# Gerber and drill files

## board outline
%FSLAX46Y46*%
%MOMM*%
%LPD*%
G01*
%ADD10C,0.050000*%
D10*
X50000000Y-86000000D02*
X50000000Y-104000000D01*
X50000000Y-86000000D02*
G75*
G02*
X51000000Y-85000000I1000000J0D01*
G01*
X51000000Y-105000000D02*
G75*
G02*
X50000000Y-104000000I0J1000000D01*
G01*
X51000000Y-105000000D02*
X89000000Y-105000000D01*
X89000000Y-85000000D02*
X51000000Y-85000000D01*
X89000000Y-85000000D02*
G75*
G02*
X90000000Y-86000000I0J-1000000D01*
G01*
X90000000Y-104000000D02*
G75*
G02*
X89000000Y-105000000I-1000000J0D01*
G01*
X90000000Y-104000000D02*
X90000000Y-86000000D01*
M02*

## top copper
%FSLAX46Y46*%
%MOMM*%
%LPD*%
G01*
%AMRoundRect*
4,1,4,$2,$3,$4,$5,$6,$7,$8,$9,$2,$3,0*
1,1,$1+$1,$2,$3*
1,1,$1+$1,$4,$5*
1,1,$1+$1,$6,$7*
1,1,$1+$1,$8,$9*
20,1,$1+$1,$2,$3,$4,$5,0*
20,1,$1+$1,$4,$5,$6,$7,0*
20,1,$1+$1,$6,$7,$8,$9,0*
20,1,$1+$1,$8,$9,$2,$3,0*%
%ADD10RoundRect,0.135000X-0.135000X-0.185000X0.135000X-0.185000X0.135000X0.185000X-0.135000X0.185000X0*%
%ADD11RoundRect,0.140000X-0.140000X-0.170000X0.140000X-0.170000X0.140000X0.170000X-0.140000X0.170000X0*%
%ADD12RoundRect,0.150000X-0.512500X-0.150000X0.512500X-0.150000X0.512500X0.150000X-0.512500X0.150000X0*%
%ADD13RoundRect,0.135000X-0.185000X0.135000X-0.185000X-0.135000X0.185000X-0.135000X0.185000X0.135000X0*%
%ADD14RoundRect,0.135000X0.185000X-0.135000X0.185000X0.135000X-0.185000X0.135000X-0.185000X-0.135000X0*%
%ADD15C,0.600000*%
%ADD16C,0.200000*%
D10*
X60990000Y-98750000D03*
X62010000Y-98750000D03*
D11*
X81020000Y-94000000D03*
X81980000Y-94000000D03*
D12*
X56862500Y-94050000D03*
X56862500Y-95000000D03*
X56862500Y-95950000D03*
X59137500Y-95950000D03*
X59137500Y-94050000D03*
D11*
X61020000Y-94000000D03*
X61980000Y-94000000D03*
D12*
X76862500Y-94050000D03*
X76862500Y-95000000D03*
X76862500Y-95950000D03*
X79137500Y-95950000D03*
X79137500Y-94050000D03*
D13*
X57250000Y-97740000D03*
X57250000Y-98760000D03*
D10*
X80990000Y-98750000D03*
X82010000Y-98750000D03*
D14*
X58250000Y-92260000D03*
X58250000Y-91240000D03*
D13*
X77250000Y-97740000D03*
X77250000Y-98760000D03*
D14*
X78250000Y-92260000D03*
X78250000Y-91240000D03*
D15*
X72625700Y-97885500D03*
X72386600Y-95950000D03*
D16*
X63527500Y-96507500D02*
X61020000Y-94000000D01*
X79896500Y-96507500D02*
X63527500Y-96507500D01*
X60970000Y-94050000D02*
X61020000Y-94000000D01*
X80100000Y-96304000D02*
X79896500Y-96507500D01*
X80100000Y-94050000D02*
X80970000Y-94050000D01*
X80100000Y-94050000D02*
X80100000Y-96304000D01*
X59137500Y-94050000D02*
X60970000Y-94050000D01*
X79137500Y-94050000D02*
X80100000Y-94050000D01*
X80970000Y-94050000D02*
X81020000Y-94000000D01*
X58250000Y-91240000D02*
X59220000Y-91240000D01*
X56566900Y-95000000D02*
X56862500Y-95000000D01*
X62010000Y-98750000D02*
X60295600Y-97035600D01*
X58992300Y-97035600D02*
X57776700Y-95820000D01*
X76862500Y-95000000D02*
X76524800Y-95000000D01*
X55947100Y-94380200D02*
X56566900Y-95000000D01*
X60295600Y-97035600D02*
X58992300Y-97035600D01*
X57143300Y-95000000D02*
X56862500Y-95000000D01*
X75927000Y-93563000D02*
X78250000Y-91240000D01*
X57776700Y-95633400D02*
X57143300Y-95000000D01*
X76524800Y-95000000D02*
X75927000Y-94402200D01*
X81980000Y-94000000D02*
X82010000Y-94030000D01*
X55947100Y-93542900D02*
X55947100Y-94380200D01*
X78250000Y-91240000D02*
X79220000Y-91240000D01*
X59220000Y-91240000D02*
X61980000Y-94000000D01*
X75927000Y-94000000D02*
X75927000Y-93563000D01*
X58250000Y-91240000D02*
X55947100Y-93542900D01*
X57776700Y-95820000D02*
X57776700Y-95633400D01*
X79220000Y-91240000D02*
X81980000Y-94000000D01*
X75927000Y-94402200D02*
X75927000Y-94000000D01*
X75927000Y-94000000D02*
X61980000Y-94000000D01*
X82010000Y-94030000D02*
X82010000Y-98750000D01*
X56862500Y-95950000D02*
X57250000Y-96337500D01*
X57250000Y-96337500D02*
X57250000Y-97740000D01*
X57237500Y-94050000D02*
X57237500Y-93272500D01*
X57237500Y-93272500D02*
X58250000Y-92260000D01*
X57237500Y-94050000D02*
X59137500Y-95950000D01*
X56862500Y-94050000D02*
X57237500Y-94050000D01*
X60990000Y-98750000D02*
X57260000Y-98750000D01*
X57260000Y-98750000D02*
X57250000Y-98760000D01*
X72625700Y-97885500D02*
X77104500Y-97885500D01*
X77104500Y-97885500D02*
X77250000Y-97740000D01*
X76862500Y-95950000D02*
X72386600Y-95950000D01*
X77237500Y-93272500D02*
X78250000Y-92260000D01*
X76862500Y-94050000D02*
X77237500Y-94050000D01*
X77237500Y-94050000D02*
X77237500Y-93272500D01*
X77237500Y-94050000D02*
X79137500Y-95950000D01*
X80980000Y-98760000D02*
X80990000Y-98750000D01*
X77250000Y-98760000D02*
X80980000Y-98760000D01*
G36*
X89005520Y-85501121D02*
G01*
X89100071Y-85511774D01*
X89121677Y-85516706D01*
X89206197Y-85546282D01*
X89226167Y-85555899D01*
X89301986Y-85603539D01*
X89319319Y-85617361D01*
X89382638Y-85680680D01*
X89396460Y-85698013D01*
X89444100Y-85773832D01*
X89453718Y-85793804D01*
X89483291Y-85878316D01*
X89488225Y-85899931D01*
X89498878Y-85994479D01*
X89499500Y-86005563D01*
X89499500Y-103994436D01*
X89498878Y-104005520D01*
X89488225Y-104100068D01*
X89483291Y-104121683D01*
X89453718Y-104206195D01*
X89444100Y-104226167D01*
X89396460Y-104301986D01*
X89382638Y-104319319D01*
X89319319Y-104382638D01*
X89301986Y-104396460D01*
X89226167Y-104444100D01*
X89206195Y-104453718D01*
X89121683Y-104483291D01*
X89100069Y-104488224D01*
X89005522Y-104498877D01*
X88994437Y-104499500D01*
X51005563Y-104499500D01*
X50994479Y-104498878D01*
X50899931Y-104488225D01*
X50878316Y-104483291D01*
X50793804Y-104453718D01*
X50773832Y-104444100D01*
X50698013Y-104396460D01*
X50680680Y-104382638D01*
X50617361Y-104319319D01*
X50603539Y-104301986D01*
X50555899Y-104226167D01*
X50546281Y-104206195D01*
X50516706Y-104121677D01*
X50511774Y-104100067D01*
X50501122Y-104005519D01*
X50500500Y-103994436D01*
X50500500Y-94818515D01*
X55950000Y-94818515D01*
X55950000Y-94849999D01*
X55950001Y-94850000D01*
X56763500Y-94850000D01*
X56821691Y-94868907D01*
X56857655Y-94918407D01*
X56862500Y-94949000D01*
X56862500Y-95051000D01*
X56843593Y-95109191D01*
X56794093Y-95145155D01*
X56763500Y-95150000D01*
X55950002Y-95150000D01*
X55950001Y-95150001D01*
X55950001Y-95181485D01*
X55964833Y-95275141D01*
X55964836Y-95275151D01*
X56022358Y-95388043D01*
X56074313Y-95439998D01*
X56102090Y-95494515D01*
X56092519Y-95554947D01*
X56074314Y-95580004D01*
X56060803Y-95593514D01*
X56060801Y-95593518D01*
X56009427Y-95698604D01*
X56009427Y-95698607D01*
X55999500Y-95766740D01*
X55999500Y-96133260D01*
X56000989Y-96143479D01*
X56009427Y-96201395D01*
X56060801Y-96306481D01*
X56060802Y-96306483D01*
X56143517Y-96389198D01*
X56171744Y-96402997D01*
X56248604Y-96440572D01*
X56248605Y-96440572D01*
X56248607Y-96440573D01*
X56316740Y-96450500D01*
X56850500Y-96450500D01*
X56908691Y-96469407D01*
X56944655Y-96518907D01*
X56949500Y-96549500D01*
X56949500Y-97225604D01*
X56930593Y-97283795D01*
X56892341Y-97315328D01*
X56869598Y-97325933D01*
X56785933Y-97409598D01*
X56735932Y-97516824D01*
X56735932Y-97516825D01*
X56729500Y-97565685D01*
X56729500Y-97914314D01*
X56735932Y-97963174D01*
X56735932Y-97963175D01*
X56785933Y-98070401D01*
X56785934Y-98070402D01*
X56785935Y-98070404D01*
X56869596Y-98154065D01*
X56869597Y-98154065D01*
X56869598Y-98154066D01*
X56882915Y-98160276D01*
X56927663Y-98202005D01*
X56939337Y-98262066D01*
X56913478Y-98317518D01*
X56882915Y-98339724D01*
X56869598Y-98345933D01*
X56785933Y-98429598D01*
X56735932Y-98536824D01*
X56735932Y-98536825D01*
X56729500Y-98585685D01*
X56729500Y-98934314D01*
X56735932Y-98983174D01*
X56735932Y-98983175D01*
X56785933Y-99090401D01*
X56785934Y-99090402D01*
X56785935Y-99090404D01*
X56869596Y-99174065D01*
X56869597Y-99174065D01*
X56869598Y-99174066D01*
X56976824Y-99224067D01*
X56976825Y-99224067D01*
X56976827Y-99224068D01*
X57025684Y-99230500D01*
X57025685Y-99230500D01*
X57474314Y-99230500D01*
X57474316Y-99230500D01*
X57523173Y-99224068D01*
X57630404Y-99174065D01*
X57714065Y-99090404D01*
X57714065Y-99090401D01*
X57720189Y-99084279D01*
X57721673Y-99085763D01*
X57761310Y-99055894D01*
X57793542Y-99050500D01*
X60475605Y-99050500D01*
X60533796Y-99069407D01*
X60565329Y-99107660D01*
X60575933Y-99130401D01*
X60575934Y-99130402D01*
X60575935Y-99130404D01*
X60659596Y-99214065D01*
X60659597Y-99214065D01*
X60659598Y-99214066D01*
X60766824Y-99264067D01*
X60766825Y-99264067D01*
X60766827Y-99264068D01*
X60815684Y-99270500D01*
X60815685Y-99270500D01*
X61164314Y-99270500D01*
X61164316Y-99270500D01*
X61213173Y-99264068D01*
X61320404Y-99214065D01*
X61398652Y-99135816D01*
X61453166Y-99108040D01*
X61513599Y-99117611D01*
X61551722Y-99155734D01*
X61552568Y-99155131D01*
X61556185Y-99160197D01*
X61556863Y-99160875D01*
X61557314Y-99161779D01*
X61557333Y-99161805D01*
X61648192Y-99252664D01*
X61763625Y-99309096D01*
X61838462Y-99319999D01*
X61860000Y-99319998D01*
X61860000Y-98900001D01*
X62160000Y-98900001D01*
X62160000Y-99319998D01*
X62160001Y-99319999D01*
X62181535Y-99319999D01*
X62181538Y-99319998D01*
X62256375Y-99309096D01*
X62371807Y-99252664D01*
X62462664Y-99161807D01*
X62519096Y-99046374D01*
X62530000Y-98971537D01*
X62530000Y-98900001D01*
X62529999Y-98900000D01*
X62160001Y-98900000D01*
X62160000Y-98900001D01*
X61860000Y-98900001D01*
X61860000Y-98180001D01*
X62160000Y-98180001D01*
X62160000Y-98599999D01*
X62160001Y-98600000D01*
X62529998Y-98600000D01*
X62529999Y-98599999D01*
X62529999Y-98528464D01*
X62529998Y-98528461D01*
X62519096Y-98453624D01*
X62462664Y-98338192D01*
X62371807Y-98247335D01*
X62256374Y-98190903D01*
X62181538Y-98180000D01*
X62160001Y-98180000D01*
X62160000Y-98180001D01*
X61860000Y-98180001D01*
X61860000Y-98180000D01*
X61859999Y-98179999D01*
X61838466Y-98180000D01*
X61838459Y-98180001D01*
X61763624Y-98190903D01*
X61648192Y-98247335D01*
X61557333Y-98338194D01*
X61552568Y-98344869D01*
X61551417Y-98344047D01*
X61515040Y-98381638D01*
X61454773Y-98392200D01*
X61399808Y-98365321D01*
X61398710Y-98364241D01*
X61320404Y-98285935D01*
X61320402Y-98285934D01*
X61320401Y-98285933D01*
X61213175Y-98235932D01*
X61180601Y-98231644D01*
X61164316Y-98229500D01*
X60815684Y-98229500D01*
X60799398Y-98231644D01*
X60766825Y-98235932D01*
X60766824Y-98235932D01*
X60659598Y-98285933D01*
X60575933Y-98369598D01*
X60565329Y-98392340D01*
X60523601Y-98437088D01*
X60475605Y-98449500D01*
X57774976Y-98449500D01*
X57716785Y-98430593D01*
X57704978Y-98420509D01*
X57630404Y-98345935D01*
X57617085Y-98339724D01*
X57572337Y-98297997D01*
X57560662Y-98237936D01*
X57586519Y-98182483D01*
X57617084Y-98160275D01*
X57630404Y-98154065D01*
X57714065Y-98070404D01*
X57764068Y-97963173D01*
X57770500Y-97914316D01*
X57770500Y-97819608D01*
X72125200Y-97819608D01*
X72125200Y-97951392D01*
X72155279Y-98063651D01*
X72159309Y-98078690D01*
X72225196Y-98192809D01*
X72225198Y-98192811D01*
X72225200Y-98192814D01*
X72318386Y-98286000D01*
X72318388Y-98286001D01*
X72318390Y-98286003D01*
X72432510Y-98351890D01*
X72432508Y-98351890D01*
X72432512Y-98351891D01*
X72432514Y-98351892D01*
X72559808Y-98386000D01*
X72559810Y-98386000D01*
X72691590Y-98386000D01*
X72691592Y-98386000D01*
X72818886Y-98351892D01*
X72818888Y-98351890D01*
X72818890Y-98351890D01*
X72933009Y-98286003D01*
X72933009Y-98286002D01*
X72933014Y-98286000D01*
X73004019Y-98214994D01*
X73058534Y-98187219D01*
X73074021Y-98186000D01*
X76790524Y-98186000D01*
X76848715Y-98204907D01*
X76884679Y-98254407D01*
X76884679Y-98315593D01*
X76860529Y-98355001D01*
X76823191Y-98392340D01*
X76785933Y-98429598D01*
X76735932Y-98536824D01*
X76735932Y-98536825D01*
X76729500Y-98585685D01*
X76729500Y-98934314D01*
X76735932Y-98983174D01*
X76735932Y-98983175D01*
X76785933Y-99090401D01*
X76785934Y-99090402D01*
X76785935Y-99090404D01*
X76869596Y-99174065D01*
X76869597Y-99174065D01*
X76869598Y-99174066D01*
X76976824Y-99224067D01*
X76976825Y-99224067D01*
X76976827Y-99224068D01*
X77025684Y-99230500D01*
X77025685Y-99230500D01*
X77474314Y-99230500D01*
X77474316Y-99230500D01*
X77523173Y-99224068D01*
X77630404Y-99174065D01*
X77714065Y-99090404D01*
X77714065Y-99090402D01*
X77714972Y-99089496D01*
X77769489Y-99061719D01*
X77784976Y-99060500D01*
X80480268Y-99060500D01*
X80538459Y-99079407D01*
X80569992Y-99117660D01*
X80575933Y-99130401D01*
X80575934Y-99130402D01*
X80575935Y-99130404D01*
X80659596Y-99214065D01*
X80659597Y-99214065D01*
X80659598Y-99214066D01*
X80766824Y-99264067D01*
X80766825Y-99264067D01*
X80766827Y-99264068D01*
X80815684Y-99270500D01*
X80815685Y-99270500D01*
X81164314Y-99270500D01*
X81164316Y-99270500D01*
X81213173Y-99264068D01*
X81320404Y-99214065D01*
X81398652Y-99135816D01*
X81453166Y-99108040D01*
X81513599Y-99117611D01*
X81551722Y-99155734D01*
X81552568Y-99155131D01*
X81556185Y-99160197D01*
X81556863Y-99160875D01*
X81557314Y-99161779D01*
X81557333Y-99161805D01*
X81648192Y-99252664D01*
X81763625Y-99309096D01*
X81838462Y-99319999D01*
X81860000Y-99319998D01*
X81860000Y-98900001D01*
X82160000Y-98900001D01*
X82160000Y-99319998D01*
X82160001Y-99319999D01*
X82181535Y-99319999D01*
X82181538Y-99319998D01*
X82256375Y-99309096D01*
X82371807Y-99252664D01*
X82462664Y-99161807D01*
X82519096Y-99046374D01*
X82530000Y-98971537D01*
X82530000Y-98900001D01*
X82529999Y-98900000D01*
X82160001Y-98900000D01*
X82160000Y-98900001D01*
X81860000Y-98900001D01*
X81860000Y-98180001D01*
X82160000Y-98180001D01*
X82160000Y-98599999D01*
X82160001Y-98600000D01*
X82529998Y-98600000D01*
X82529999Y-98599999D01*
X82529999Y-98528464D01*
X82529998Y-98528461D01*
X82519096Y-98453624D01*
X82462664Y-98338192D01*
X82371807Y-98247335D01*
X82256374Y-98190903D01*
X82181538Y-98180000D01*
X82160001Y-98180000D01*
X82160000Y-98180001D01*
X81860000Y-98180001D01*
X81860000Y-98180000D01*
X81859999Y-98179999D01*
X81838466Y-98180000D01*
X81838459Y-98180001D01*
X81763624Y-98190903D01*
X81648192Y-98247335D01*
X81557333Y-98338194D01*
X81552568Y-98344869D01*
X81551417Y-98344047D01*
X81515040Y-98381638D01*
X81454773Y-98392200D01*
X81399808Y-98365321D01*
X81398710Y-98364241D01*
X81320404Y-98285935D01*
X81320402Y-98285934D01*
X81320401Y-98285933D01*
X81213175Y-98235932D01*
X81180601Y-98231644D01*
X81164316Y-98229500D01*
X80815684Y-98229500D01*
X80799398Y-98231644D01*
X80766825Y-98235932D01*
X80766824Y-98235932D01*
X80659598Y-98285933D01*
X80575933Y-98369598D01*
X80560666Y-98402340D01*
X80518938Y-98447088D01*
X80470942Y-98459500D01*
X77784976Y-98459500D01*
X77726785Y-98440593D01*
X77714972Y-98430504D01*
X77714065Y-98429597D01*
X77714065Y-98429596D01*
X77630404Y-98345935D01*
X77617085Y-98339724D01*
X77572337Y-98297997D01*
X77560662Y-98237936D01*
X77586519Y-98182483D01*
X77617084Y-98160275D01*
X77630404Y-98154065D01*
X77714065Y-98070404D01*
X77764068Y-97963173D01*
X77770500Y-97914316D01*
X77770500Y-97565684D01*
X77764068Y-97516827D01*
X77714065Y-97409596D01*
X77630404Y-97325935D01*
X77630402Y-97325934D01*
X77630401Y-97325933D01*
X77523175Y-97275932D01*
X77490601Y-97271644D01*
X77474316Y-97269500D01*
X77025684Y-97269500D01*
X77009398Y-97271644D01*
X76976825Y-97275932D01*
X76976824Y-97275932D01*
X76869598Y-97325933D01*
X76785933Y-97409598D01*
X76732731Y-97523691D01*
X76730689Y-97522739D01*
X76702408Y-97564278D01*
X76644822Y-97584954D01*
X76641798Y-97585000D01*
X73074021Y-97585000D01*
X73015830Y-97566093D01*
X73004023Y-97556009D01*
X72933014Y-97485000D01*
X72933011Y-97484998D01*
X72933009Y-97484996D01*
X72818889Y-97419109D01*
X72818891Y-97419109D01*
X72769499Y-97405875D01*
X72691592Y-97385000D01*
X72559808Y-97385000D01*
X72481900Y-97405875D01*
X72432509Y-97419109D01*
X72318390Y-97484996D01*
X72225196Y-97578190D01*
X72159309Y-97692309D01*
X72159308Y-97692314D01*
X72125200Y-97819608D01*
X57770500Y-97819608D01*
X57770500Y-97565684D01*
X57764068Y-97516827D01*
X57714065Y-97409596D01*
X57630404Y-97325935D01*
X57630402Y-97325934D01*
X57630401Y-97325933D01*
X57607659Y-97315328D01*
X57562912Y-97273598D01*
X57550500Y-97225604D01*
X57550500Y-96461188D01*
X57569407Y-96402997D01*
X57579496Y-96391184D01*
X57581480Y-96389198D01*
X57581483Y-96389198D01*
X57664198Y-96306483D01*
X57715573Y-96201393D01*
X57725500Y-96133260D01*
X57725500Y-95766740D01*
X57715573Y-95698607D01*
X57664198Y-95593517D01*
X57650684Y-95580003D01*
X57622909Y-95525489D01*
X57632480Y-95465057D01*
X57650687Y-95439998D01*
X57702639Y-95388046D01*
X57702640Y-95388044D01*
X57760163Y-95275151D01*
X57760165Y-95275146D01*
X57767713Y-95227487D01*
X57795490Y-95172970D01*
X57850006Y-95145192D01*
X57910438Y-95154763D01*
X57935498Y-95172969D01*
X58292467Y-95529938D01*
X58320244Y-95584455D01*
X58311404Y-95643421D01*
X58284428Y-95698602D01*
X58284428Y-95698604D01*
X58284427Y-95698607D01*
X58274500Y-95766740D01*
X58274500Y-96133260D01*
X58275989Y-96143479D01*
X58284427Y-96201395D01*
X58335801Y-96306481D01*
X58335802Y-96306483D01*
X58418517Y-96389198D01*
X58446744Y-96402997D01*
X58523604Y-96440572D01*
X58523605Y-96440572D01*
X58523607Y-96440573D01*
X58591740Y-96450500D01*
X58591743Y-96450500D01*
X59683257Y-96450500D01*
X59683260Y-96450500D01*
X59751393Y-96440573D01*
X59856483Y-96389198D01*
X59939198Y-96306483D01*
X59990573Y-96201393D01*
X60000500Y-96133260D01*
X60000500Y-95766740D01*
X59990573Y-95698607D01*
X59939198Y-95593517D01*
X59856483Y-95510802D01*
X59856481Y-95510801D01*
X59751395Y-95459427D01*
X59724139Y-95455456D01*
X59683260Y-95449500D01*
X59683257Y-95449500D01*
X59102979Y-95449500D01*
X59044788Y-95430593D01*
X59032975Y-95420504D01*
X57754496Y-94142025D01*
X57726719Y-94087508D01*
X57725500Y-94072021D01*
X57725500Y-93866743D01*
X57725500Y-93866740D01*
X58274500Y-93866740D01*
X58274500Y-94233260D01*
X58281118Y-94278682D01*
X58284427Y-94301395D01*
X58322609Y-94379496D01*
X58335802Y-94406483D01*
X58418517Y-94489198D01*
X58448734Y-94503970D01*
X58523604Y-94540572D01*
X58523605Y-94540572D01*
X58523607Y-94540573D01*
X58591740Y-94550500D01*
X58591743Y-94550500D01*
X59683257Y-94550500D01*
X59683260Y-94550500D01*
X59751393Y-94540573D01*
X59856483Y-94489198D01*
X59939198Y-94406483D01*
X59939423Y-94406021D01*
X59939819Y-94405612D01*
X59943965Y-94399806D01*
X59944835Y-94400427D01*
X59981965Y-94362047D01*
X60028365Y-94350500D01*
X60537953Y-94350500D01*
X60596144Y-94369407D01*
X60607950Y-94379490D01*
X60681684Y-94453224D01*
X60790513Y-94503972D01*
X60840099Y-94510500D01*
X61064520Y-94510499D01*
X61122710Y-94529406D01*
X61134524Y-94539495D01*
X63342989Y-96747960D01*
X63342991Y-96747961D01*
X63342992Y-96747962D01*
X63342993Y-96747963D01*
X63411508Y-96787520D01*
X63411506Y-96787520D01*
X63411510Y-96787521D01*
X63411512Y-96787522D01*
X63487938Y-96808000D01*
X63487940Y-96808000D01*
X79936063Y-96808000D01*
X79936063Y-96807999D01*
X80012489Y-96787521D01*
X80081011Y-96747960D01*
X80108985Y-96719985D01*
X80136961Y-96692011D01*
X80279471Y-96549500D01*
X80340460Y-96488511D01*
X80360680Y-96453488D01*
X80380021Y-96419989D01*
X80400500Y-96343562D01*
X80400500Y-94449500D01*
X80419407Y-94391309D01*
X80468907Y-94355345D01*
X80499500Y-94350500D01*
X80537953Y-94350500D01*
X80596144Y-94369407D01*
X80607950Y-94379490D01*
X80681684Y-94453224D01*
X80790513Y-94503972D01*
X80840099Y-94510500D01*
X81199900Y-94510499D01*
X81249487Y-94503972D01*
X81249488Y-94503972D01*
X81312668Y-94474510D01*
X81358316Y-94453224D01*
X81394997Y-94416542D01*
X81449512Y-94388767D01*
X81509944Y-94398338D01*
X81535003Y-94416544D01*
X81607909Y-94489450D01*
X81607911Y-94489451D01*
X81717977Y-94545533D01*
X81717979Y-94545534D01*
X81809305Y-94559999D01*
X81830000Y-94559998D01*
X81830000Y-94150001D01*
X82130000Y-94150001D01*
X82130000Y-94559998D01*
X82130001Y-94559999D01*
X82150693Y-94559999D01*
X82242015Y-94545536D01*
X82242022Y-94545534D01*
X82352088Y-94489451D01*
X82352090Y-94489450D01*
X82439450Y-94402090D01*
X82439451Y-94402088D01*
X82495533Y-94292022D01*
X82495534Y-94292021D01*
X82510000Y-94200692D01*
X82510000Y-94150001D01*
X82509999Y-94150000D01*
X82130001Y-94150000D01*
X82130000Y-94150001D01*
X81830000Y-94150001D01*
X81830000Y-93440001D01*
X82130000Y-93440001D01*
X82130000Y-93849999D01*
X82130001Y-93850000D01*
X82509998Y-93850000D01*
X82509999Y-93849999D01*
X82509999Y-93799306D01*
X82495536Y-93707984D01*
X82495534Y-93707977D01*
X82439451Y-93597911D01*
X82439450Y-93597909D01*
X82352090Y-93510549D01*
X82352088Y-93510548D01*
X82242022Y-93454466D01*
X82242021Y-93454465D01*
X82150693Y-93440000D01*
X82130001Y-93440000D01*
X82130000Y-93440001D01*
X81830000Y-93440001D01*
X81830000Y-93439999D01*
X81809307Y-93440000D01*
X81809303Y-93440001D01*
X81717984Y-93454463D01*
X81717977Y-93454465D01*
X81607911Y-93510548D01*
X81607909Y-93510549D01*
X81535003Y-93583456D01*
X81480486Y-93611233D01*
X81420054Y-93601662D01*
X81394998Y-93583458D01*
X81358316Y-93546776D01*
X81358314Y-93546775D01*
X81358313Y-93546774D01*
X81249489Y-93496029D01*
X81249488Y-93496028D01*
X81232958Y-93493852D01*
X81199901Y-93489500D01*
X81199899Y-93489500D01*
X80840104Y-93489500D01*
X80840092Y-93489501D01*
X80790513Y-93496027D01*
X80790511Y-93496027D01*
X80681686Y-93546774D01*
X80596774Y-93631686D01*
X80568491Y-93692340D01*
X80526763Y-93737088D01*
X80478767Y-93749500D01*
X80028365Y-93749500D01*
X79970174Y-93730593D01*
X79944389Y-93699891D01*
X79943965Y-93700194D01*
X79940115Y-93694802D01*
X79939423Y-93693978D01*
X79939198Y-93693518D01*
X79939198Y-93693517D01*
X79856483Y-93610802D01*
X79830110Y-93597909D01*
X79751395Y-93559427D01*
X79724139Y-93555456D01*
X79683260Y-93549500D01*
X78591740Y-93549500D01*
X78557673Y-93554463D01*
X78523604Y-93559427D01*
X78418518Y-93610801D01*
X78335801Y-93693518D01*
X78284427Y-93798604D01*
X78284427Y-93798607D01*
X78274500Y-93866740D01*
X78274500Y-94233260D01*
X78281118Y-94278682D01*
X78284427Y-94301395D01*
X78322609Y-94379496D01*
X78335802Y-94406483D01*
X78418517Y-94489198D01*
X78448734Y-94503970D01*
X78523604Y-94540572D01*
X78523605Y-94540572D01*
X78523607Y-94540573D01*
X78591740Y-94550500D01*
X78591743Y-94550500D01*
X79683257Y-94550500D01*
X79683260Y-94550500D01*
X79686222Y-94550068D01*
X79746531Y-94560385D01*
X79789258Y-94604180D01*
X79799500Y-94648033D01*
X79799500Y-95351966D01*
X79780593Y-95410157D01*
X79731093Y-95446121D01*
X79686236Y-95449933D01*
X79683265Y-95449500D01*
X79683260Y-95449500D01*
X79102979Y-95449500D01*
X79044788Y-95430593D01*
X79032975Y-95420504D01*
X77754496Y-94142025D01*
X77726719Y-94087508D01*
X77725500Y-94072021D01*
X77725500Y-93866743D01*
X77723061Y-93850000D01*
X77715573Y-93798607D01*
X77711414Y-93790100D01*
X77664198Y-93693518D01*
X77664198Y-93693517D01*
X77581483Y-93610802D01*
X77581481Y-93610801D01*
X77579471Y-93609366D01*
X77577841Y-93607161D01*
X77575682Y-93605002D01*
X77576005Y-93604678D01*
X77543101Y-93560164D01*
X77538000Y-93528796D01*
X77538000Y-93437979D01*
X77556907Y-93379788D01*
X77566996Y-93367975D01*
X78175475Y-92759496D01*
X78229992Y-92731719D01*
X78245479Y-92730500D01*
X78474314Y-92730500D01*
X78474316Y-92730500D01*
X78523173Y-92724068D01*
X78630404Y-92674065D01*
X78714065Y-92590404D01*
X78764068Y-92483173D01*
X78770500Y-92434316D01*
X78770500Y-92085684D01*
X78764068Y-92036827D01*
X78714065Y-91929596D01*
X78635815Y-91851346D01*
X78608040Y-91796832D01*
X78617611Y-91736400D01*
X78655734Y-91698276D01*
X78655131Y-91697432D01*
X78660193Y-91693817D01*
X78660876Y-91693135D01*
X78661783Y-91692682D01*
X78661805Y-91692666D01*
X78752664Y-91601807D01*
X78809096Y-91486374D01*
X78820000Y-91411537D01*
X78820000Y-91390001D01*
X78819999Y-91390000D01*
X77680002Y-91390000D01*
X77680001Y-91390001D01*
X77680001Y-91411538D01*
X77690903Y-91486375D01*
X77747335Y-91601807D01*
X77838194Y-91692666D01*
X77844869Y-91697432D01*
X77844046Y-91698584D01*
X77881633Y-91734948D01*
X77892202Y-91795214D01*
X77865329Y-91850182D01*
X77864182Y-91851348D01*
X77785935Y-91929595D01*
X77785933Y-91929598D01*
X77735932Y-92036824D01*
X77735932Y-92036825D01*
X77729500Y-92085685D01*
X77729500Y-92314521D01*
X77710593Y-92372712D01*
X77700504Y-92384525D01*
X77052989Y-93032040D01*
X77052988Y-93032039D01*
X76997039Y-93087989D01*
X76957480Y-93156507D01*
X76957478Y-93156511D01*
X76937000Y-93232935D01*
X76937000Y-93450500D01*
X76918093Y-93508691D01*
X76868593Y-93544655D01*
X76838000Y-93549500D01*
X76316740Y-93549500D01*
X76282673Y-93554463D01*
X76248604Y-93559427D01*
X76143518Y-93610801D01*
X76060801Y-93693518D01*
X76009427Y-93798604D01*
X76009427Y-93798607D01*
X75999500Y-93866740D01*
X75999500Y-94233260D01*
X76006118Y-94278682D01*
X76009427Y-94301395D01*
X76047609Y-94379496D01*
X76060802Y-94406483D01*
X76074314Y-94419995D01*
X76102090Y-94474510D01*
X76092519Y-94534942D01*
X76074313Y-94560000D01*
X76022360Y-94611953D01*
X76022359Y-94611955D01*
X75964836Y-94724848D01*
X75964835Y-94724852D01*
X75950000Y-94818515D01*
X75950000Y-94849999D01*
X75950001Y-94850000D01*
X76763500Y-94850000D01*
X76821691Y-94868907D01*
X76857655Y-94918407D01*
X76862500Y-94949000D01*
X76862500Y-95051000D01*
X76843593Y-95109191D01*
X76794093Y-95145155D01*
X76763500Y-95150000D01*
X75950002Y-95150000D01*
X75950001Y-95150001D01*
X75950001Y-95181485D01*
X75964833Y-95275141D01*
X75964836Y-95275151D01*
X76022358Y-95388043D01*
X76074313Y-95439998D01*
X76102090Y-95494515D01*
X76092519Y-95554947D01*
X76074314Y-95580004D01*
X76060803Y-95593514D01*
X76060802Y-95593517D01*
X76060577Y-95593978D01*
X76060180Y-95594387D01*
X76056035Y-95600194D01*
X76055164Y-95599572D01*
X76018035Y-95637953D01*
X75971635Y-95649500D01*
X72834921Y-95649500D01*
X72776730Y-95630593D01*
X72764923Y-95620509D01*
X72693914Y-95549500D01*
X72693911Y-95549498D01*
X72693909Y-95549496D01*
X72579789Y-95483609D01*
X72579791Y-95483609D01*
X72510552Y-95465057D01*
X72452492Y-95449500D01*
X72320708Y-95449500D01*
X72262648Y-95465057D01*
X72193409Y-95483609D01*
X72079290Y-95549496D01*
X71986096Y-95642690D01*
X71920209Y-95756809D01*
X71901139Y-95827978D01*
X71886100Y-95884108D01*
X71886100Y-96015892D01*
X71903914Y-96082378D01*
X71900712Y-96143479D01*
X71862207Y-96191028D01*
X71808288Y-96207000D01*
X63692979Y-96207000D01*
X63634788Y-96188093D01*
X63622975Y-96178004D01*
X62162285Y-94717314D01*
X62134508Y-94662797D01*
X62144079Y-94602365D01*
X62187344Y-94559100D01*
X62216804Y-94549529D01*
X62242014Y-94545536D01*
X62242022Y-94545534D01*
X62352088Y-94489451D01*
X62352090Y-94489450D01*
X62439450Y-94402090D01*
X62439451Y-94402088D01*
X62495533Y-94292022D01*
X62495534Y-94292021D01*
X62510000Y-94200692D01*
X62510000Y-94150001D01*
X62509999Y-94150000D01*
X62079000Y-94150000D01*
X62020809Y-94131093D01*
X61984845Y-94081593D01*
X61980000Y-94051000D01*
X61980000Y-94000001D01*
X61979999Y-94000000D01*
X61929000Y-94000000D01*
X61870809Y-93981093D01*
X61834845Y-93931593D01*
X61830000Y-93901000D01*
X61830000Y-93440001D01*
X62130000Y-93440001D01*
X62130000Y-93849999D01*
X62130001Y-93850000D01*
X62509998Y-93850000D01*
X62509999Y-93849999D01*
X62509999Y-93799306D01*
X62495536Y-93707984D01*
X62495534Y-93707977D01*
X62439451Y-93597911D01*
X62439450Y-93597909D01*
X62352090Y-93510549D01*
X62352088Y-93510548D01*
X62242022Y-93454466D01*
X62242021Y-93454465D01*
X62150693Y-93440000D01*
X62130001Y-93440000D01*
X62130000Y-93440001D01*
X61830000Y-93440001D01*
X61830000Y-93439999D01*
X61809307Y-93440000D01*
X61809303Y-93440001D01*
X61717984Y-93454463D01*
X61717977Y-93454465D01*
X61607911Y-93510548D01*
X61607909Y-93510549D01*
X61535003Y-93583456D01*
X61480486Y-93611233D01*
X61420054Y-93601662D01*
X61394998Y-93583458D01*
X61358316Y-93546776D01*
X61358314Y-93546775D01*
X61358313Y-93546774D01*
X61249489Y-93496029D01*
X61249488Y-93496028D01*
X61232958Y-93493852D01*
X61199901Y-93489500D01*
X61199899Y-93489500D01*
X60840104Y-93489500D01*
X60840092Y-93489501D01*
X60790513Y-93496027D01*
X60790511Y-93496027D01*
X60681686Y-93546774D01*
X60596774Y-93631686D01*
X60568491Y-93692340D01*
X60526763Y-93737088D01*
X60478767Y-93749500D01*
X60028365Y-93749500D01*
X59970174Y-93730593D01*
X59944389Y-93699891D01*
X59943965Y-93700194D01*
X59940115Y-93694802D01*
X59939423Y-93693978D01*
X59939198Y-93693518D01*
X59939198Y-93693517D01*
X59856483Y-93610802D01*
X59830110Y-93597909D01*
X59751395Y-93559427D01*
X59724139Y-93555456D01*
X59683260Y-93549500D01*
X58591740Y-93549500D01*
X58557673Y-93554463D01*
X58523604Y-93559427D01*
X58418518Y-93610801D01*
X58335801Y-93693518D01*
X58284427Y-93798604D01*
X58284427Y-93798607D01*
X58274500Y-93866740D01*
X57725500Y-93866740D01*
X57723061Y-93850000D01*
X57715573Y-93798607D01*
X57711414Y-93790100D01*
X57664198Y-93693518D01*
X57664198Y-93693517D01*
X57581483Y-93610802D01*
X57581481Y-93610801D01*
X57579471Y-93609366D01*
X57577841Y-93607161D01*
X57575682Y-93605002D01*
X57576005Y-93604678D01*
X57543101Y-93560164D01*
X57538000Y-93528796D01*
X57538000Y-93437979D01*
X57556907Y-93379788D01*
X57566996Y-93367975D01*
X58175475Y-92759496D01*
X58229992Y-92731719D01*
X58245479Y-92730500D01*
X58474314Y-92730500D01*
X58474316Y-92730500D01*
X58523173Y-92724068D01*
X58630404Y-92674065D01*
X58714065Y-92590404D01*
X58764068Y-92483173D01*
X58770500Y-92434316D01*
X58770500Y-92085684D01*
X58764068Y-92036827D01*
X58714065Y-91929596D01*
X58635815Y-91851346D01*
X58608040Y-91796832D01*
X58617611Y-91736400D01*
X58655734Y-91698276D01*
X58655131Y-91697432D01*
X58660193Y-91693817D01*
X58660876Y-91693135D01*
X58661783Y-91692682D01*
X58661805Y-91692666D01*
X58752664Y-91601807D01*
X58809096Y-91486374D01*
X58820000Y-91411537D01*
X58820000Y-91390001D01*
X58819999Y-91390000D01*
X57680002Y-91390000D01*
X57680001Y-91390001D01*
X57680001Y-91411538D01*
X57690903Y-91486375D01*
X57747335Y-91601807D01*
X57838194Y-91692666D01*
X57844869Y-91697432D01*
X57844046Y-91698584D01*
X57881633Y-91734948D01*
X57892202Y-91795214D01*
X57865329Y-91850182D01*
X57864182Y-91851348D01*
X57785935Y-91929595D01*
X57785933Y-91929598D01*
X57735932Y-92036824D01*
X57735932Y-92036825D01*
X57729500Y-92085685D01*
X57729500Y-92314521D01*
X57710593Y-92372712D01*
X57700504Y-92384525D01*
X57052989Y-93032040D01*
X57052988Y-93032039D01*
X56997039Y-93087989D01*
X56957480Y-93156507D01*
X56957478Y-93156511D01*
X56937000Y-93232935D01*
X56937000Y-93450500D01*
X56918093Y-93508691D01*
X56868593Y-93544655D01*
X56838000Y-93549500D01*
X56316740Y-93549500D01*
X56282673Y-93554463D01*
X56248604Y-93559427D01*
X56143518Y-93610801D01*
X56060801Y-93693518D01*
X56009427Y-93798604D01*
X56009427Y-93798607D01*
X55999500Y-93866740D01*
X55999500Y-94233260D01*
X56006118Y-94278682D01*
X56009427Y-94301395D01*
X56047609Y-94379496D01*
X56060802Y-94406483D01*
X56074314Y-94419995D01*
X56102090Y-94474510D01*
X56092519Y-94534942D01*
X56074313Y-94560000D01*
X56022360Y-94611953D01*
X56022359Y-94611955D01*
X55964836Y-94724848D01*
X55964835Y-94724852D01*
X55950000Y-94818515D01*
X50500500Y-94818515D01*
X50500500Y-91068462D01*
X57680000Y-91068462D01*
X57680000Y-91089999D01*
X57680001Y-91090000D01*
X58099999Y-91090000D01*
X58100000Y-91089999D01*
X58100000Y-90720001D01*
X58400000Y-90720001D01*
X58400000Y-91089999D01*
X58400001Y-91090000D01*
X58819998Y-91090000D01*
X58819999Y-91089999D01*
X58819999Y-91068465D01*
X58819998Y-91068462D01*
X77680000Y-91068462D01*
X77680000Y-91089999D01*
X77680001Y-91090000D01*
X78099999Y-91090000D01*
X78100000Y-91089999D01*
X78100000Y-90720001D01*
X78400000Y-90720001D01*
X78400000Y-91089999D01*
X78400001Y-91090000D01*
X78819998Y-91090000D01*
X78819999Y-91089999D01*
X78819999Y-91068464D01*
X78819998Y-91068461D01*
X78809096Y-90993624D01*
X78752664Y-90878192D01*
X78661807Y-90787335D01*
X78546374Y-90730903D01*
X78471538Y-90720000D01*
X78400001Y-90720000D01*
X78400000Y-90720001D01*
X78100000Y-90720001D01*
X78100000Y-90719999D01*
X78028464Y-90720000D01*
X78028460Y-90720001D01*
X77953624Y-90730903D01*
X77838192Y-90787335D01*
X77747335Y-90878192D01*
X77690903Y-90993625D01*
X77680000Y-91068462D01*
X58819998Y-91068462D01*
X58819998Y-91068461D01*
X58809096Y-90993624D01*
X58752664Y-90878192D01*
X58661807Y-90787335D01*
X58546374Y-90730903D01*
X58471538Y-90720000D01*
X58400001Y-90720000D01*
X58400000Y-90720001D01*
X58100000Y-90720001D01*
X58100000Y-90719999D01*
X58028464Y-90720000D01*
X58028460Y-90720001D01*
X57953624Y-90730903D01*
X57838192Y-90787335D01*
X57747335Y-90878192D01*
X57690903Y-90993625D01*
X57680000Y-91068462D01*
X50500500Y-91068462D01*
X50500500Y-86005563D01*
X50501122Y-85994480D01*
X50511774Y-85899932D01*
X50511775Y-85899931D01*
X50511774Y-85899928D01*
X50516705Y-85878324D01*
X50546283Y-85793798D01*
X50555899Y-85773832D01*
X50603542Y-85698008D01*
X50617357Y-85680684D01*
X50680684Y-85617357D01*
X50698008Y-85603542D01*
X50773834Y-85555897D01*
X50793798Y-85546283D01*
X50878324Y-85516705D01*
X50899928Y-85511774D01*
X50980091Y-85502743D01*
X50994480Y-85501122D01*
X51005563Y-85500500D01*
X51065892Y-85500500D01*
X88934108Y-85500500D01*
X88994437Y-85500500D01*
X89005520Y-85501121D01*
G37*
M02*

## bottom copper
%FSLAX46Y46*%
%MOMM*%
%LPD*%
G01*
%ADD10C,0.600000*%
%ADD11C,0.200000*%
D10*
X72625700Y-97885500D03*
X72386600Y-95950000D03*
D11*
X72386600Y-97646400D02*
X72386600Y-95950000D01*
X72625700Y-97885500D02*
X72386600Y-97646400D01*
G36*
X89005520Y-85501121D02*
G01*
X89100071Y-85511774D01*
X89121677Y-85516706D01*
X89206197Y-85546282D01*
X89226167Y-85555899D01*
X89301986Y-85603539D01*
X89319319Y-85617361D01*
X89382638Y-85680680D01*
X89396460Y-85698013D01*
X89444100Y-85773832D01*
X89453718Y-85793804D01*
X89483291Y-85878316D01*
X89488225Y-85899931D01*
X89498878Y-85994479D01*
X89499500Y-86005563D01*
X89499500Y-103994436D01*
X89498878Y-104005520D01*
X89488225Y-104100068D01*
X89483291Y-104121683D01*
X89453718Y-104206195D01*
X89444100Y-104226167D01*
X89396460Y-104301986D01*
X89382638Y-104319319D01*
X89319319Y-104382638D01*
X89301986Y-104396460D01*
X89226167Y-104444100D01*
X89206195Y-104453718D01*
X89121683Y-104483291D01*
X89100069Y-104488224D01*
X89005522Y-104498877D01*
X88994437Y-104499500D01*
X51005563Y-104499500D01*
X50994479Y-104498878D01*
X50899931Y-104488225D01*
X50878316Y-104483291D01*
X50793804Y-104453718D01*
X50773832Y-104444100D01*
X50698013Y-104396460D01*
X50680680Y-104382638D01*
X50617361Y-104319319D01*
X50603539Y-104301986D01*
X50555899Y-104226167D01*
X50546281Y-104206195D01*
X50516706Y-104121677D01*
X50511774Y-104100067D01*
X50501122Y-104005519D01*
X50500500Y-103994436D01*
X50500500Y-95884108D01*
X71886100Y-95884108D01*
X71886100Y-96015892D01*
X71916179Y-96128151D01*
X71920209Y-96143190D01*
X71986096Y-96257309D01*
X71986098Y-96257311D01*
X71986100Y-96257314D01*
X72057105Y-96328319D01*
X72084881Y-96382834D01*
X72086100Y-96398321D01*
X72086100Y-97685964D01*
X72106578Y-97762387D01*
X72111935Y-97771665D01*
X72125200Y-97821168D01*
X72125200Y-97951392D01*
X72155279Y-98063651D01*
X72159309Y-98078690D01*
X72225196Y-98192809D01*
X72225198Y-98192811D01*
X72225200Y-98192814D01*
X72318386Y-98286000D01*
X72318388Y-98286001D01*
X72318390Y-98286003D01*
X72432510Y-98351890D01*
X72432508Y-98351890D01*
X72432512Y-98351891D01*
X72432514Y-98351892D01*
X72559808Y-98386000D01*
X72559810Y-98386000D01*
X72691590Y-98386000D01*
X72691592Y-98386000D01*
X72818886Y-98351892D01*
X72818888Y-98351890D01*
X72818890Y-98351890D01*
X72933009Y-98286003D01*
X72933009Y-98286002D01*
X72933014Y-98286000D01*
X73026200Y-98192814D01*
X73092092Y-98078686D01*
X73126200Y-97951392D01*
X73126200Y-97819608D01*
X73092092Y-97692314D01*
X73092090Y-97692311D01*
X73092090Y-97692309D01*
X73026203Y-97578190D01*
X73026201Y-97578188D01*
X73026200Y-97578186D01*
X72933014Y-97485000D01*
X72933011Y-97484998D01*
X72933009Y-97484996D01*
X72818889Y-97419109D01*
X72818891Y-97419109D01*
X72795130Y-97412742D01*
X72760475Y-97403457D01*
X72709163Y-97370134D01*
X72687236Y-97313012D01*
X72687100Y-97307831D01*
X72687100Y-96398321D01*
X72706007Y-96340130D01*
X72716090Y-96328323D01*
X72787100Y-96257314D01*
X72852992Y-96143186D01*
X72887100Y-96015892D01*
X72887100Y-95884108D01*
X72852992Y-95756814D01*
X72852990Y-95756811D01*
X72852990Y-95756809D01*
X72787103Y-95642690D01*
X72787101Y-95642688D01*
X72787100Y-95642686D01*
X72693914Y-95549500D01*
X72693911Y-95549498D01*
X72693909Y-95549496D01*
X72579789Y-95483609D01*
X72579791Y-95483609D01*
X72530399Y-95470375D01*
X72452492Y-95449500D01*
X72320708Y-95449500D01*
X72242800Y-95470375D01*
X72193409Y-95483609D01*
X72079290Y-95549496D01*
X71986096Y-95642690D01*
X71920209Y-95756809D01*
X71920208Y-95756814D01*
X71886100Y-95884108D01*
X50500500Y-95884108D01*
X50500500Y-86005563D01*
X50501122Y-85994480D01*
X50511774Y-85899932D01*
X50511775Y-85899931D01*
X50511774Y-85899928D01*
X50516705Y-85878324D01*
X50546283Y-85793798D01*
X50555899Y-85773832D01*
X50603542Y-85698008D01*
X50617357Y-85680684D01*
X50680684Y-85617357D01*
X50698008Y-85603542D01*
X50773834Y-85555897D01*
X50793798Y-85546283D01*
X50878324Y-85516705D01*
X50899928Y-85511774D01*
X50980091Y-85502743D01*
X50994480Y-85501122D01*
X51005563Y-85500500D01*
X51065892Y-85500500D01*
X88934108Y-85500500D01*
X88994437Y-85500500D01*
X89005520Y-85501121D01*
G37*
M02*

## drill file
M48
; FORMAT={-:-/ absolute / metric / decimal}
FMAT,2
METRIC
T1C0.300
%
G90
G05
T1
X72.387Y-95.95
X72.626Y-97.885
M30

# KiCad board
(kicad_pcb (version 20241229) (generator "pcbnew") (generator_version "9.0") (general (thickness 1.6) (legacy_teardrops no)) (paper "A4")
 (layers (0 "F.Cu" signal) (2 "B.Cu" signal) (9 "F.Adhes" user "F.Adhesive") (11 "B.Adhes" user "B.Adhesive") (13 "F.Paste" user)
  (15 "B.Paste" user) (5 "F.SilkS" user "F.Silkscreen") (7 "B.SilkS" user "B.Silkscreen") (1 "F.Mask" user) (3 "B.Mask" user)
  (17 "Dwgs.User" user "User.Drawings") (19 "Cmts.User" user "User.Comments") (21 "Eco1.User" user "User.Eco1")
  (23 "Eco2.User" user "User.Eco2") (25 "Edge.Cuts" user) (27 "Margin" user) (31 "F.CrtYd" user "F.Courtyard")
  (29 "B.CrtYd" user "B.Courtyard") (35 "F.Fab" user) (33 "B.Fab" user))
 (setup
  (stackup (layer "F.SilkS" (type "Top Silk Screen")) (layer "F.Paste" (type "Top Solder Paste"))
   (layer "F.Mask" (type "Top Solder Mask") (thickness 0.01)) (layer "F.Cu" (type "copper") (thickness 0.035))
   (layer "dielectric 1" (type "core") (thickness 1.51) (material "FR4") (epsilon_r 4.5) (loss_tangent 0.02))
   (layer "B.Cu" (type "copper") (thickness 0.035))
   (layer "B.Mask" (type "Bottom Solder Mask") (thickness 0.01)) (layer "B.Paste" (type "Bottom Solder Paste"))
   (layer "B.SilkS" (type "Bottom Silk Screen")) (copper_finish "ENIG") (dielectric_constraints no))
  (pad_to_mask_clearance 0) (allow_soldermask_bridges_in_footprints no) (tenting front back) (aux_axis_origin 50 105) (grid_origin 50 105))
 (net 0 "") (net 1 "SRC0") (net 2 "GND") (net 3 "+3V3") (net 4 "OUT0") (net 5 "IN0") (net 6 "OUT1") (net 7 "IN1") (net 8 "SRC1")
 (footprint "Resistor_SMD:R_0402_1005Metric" (layer "F.Cu") (at 61.5 98.75)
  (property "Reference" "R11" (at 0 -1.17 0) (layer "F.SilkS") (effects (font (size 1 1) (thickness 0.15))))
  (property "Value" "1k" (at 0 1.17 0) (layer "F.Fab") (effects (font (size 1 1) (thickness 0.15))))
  (pad "1" smd roundrect (at -0.51 0) (size 0.54 0.64) (layers "F.Cu" "F.Mask" "F.Paste") (roundrect_rratio 0.25) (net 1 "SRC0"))
  (pad "2" smd roundrect (at 0.51 0) (size 0.54 0.64) (layers "F.Cu" "F.Mask" "F.Paste") (roundrect_rratio 0.25) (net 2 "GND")))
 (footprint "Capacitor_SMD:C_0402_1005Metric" (layer "F.Cu") (at 81.5 94)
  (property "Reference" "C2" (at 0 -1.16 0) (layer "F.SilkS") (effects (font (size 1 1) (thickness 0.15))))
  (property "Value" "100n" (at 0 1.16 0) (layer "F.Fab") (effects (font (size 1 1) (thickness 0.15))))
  (pad "1" smd roundrect (at -0.48 0) (size 0.56 0.62) (layers "F.Cu" "F.Mask" "F.Paste") (roundrect_rratio 0.25) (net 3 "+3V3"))
  (pad "2" smd roundrect (at 0.48 0) (size 0.56 0.62) (layers "F.Cu" "F.Mask" "F.Paste") (roundrect_rratio 0.25) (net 2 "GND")))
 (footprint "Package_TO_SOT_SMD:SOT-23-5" (layer "F.Cu") (at 58 95)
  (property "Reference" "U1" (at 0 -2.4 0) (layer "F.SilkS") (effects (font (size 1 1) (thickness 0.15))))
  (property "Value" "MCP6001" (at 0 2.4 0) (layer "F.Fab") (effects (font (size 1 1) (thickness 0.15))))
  (pad "1" smd roundrect (at -1.1375 -0.95) (size 1.325 0.6) (layers "F.Cu" "F.Mask" "F.Paste") (roundrect_rratio 0.25) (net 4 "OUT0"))
  (pad "2" smd roundrect (at -1.1375 0) (size 1.325 0.6) (layers "F.Cu" "F.Mask" "F.Paste") (roundrect_rratio 0.25) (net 2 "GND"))
  (pad "3" smd roundrect (at -1.1375 0.95) (size 1.325 0.6) (layers "F.Cu" "F.Mask" "F.Paste") (roundrect_rratio 0.25) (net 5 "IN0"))
  (pad "4" smd roundrect (at 1.1375 0.95) (size 1.325 0.6) (layers "F.Cu" "F.Mask" "F.Paste") (roundrect_rratio 0.25) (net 4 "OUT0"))
  (pad "5" smd roundrect (at 1.1375 -0.95) (size 1.325 0.6) (layers "F.Cu" "F.Mask" "F.Paste") (roundrect_rratio 0.25) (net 3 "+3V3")))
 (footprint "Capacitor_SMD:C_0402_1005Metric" (layer "F.Cu") (at 61.5 94)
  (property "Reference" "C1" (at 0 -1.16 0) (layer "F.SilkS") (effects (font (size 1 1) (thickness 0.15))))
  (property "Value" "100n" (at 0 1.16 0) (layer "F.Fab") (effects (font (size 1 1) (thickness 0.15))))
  (pad "1" smd roundrect (at -0.48 0) (size 0.56 0.62) (layers "F.Cu" "F.Mask" "F.Paste") (roundrect_rratio 0.25) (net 3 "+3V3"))
  (pad "2" smd roundrect (at 0.48 0) (size 0.56 0.62) (layers "F.Cu" "F.Mask" "F.Paste") (roundrect_rratio 0.25) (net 2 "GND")))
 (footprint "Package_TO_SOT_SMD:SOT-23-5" (layer "F.Cu") (at 78 95)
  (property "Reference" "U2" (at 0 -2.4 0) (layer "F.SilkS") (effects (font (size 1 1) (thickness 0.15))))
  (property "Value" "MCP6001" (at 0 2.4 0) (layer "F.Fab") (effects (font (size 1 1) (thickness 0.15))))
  (pad "1" smd roundrect (at -1.1375 -0.95) (size 1.325 0.6) (layers "F.Cu" "F.Mask" "F.Paste") (roundrect_rratio 0.25) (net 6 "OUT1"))
  (pad "2" smd roundrect (at -1.1375 0) (size 1.325 0.6) (layers "F.Cu" "F.Mask" "F.Paste") (roundrect_rratio 0.25) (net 2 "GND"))
  (pad "3" smd roundrect (at -1.1375 0.95) (size 1.325 0.6) (layers "F.Cu" "F.Mask" "F.Paste") (roundrect_rratio 0.25) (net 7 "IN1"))
  (pad "4" smd roundrect (at 1.1375 0.95) (size 1.325 0.6) (layers "F.Cu" "F.Mask" "F.Paste") (roundrect_rratio 0.25) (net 6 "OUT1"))
  (pad "5" smd roundrect (at 1.1375 -0.95) (size 1.325 0.6) (layers "F.Cu" "F.Mask" "F.Paste") (roundrect_rratio 0.25) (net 3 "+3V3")))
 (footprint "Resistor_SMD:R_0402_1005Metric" (layer "F.Cu") (at 57.25 98.25 -90)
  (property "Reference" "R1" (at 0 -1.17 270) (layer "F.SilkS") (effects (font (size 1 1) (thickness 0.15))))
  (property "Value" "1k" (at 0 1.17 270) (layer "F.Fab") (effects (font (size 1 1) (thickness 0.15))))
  (pad "1" smd roundrect (at -0.51 0 270) (size 0.54 0.64) (layers "F.Cu" "F.Mask" "F.Paste") (roundrect_rratio 0.25) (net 5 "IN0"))
  (pad "2" smd roundrect (at 0.51 0 270) (size 0.54 0.64) (layers "F.Cu" "F.Mask" "F.Paste") (roundrect_rratio 0.25) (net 1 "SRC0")))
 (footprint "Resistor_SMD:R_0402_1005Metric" (layer "F.Cu") (at 81.5 98.75)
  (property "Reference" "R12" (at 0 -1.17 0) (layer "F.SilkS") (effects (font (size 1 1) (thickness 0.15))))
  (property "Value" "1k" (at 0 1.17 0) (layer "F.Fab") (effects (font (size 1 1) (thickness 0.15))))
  (pad "1" smd roundrect (at -0.51 0) (size 0.54 0.64) (layers "F.Cu" "F.Mask" "F.Paste") (roundrect_rratio 0.25) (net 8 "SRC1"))
  (pad "2" smd roundrect (at 0.51 0) (size 0.54 0.64) (layers "F.Cu" "F.Mask" "F.Paste") (roundrect_rratio 0.25) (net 2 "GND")))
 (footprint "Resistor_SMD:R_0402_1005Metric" (layer "F.Cu") (at 58.25 91.75 90)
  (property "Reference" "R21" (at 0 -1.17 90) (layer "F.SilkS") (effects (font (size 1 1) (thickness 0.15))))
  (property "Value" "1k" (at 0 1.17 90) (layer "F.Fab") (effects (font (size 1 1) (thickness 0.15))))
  (pad "1" smd roundrect (at -0.51 0 90) (size 0.54 0.64) (layers "F.Cu" "F.Mask" "F.Paste") (roundrect_rratio 0.25) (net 4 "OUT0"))
  (pad "2" smd roundrect (at 0.51 0 90) (size 0.54 0.64) (layers "F.Cu" "F.Mask" "F.Paste") (roundrect_rratio 0.25) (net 2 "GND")))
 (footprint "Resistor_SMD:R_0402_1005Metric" (layer "F.Cu") (at 77.25 98.25 -90)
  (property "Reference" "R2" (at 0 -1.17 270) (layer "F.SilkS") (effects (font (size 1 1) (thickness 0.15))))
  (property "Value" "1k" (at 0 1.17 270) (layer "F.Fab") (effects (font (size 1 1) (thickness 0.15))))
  (pad "1" smd roundrect (at -0.51 0 270) (size 0.54 0.64) (layers "F.Cu" "F.Mask" "F.Paste") (roundrect_rratio 0.25) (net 7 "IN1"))
  (pad "2" smd roundrect (at 0.51 0 270) (size 0.54 0.64) (layers "F.Cu" "F.Mask" "F.Paste") (roundrect_rratio 0.25) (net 8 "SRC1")))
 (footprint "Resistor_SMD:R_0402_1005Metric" (layer "F.Cu") (at 78.25 91.75 90)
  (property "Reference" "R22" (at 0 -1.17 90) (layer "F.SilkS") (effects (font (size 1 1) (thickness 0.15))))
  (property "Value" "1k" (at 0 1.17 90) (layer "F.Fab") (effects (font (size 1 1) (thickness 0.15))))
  (pad "1" smd roundrect (at -0.51 0 90) (size 0.54 0.64) (layers "F.Cu" "F.Mask" "F.Paste") (roundrect_rratio 0.25) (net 6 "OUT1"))
  (pad "2" smd roundrect (at 0.51 0 90) (size 0.54 0.64) (layers "F.Cu" "F.Mask" "F.Paste") (roundrect_rratio 0.25) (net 2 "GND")))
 (gr_line (start 50 86) (end 50 104) (stroke (width 0.05) (type default)) (layer "Edge.Cuts"))
 (gr_arc (start 50 86) (mid 50.292893 85.292893) (end 51 85) (stroke (width 0.05) (type default)) (layer "Edge.Cuts"))
 (gr_arc (start 51 105) (mid 50.292893 104.707107) (end 50 104) (stroke (width 0.05) (type default)) (layer "Edge.Cuts"))
 (gr_line (start 51 105) (end 89 105) (stroke (width 0.05) (type default)) (layer "Edge.Cuts"))
 (gr_line (start 89 85) (end 51 85) (stroke (width 0.05) (type default)) (layer "Edge.Cuts"))
 (gr_arc (start 89 85) (mid 89.707107 85.292893) (end 90 86) (stroke (width 0.05) (type default)) (layer "Edge.Cuts"))
 (gr_arc (start 90 104) (mid 89.707107 104.707107) (end 89 105) (stroke (width 0.05) (type default)) (layer "Edge.Cuts"))
 (gr_line (start 90 104) (end 90 86) (stroke (width 0.05) (type default)) (layer "Edge.Cuts"))
 (segment (start 63.5275 96.5075) (end 61.02 94) (width 0.2) (layer "F.Cu") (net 3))
 (segment (start 79.8965 96.5075) (end 63.5275 96.5075) (width 0.2) (layer "F.Cu") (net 3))
 (segment (start 60.97 94.05) (end 61.02 94) (width 0.2) (layer "F.Cu") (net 3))
 (segment (start 80.1 96.304) (end 79.8965 96.5075) (width 0.2) (layer "F.Cu") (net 3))
 (segment (start 80.1 94.05) (end 80.97 94.05) (width 0.2) (layer "F.Cu") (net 3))
 (segment (start 80.1 94.05) (end 80.1 96.304) (width 0.2) (layer "F.Cu") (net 3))
 (segment (start 59.1375 94.05) (end 60.97 94.05) (width 0.2) (layer "F.Cu") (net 3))
 (segment (start 79.1375 94.05) (end 80.1 94.05) (width 0.2) (layer "F.Cu") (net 3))
 (segment (start 80.97 94.05) (end 81.02 94) (width 0.2) (layer "F.Cu") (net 3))
 (segment (start 58.25 91.24) (end 59.22 91.24) (width 0.2) (layer "F.Cu") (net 2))
 (segment (start 56.5669 95) (end 56.8625 95) (width 0.2) (layer "F.Cu") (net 2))
 (segment (start 62.01 98.75) (end 60.2956 97.0356) (width 0.2) (layer "F.Cu") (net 2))
 (segment (start 58.9923 97.0356) (end 57.7767 95.82) (width 0.2) (layer "F.Cu") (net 2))
 (segment (start 76.8625 95) (end 76.5248 95) (width 0.2) (layer "F.Cu") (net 2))
 (segment (start 55.9471 94.3802) (end 56.5669 95) (width 0.2) (layer "F.Cu") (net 2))
 (segment (start 60.2956 97.0356) (end 58.9923 97.0356) (width 0.2) (layer "F.Cu") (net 2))
 (segment (start 57.1433 95) (end 56.8625 95) (width 0.2) (layer "F.Cu") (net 2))
 (segment (start 75.927 93.563) (end 78.25 91.24) (width 0.2) (layer "F.Cu") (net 2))
 (segment (start 57.7767 95.6334) (end 57.1433 95) (width 0.2) (layer "F.Cu") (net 2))
 (segment (start 76.5248 95) (end 75.927 94.4022) (width 0.2) (layer "F.Cu") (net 2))
 (segment (start 81.98 94) (end 82.01 94.03) (width 0.2) (layer "F.Cu") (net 2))
 (segment (start 55.9471 93.5429) (end 55.9471 94.3802) (width 0.2) (layer "F.Cu") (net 2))
 (segment (start 78.25 91.24) (end 79.22 91.24) (width 0.2) (layer "F.Cu") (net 2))
 (segment (start 59.22 91.24) (end 61.98 94) (width 0.2) (layer "F.Cu") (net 2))
 (segment (start 75.927 94) (end 75.927 93.563) (width 0.2) (layer "F.Cu") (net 2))
 (segment (start 58.25 91.24) (end 55.9471 93.5429) (width 0.2) (layer "F.Cu") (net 2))
 (segment (start 57.7767 95.82) (end 57.7767 95.6334) (width 0.2) (layer "F.Cu") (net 2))
 (segment (start 79.22 91.24) (end 81.98 94) (width 0.2) (layer "F.Cu") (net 2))
 (segment (start 75.927 94.4022) (end 75.927 94) (width 0.2) (layer "F.Cu") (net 2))
 (segment (start 75.927 94) (end 61.98 94) (width 0.2) (layer "F.Cu") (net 2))
 (segment (start 82.01 94.03) (end 82.01 98.75) (width 0.2) (layer "F.Cu") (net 2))
 (segment (start 56.8625 95.95) (end 57.25 96.3375) (width 0.2) (layer "F.Cu") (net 5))
 (segment (start 57.25 96.3375) (end 57.25 97.74) (width 0.2) (layer "F.Cu") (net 5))
 (segment (start 57.2375 94.05) (end 57.2375 93.2725) (width 0.2) (layer "F.Cu") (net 4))
 (segment (start 57.2375 93.2725) (end 58.25 92.26) (width 0.2) (layer "F.Cu") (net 4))
 (segment (start 57.2375 94.05) (end 59.1375 95.95) (width 0.2) (layer "F.Cu") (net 4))
 (segment (start 56.8625 94.05) (end 57.2375 94.05) (width 0.2) (layer "F.Cu") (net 4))
 (segment (start 60.99 98.75) (end 57.26 98.75) (width 0.2) (layer "F.Cu") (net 1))
 (segment (start 57.26 98.75) (end 57.25 98.76) (width 0.2) (layer "F.Cu") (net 1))
 (segment (start 72.6257 97.8855) (end 77.1045 97.8855) (width 0.2) (layer "F.Cu") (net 7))
 (segment (start 77.1045 97.8855) (end 77.25 97.74) (width 0.2) (layer "F.Cu") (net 7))
 (segment (start 76.8625 95.95) (end 72.3866 95.95) (width 0.2) (layer "F.Cu") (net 7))
 (via (at 72.6257 97.8855) (size 0.6) (drill 0.3) (layers "F.Cu" "B.Cu") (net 7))
 (via (at 72.3866 95.95) (size 0.6) (drill 0.3) (layers "F.Cu" "B.Cu") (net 7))
 (segment (start 72.3866 97.6464) (end 72.3866 95.95) (width 0.2) (layer "B.Cu") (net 7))
 (segment (start 72.6257 97.8855) (end 72.3866 97.6464) (width 0.2) (layer "B.Cu") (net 7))
 (segment (start 77.2375 93.2725) (end 78.25 92.26) (width 0.2) (layer "F.Cu") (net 6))
 (segment (start 76.8625 94.05) (end 77.2375 94.05) (width 0.2) (layer "F.Cu") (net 6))
 (segment (start 77.2375 94.05) (end 77.2375 93.2725) (width 0.2) (layer "F.Cu") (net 6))
 (segment (start 77.2375 94.05) (end 79.1375 95.95) (width 0.2) (layer "F.Cu") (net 6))
 (segment (start 80.98 98.76) (end 80.99 98.75) (width 0.2) (layer "F.Cu") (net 8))
 (segment (start 77.25 98.76) (end 80.98 98.76) (width 0.2) (layer "F.Cu") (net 8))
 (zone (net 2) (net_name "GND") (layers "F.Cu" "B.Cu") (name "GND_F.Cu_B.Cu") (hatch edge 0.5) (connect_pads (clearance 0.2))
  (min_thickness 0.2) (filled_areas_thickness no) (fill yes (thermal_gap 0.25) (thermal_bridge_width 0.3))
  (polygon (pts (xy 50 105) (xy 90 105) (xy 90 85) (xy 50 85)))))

